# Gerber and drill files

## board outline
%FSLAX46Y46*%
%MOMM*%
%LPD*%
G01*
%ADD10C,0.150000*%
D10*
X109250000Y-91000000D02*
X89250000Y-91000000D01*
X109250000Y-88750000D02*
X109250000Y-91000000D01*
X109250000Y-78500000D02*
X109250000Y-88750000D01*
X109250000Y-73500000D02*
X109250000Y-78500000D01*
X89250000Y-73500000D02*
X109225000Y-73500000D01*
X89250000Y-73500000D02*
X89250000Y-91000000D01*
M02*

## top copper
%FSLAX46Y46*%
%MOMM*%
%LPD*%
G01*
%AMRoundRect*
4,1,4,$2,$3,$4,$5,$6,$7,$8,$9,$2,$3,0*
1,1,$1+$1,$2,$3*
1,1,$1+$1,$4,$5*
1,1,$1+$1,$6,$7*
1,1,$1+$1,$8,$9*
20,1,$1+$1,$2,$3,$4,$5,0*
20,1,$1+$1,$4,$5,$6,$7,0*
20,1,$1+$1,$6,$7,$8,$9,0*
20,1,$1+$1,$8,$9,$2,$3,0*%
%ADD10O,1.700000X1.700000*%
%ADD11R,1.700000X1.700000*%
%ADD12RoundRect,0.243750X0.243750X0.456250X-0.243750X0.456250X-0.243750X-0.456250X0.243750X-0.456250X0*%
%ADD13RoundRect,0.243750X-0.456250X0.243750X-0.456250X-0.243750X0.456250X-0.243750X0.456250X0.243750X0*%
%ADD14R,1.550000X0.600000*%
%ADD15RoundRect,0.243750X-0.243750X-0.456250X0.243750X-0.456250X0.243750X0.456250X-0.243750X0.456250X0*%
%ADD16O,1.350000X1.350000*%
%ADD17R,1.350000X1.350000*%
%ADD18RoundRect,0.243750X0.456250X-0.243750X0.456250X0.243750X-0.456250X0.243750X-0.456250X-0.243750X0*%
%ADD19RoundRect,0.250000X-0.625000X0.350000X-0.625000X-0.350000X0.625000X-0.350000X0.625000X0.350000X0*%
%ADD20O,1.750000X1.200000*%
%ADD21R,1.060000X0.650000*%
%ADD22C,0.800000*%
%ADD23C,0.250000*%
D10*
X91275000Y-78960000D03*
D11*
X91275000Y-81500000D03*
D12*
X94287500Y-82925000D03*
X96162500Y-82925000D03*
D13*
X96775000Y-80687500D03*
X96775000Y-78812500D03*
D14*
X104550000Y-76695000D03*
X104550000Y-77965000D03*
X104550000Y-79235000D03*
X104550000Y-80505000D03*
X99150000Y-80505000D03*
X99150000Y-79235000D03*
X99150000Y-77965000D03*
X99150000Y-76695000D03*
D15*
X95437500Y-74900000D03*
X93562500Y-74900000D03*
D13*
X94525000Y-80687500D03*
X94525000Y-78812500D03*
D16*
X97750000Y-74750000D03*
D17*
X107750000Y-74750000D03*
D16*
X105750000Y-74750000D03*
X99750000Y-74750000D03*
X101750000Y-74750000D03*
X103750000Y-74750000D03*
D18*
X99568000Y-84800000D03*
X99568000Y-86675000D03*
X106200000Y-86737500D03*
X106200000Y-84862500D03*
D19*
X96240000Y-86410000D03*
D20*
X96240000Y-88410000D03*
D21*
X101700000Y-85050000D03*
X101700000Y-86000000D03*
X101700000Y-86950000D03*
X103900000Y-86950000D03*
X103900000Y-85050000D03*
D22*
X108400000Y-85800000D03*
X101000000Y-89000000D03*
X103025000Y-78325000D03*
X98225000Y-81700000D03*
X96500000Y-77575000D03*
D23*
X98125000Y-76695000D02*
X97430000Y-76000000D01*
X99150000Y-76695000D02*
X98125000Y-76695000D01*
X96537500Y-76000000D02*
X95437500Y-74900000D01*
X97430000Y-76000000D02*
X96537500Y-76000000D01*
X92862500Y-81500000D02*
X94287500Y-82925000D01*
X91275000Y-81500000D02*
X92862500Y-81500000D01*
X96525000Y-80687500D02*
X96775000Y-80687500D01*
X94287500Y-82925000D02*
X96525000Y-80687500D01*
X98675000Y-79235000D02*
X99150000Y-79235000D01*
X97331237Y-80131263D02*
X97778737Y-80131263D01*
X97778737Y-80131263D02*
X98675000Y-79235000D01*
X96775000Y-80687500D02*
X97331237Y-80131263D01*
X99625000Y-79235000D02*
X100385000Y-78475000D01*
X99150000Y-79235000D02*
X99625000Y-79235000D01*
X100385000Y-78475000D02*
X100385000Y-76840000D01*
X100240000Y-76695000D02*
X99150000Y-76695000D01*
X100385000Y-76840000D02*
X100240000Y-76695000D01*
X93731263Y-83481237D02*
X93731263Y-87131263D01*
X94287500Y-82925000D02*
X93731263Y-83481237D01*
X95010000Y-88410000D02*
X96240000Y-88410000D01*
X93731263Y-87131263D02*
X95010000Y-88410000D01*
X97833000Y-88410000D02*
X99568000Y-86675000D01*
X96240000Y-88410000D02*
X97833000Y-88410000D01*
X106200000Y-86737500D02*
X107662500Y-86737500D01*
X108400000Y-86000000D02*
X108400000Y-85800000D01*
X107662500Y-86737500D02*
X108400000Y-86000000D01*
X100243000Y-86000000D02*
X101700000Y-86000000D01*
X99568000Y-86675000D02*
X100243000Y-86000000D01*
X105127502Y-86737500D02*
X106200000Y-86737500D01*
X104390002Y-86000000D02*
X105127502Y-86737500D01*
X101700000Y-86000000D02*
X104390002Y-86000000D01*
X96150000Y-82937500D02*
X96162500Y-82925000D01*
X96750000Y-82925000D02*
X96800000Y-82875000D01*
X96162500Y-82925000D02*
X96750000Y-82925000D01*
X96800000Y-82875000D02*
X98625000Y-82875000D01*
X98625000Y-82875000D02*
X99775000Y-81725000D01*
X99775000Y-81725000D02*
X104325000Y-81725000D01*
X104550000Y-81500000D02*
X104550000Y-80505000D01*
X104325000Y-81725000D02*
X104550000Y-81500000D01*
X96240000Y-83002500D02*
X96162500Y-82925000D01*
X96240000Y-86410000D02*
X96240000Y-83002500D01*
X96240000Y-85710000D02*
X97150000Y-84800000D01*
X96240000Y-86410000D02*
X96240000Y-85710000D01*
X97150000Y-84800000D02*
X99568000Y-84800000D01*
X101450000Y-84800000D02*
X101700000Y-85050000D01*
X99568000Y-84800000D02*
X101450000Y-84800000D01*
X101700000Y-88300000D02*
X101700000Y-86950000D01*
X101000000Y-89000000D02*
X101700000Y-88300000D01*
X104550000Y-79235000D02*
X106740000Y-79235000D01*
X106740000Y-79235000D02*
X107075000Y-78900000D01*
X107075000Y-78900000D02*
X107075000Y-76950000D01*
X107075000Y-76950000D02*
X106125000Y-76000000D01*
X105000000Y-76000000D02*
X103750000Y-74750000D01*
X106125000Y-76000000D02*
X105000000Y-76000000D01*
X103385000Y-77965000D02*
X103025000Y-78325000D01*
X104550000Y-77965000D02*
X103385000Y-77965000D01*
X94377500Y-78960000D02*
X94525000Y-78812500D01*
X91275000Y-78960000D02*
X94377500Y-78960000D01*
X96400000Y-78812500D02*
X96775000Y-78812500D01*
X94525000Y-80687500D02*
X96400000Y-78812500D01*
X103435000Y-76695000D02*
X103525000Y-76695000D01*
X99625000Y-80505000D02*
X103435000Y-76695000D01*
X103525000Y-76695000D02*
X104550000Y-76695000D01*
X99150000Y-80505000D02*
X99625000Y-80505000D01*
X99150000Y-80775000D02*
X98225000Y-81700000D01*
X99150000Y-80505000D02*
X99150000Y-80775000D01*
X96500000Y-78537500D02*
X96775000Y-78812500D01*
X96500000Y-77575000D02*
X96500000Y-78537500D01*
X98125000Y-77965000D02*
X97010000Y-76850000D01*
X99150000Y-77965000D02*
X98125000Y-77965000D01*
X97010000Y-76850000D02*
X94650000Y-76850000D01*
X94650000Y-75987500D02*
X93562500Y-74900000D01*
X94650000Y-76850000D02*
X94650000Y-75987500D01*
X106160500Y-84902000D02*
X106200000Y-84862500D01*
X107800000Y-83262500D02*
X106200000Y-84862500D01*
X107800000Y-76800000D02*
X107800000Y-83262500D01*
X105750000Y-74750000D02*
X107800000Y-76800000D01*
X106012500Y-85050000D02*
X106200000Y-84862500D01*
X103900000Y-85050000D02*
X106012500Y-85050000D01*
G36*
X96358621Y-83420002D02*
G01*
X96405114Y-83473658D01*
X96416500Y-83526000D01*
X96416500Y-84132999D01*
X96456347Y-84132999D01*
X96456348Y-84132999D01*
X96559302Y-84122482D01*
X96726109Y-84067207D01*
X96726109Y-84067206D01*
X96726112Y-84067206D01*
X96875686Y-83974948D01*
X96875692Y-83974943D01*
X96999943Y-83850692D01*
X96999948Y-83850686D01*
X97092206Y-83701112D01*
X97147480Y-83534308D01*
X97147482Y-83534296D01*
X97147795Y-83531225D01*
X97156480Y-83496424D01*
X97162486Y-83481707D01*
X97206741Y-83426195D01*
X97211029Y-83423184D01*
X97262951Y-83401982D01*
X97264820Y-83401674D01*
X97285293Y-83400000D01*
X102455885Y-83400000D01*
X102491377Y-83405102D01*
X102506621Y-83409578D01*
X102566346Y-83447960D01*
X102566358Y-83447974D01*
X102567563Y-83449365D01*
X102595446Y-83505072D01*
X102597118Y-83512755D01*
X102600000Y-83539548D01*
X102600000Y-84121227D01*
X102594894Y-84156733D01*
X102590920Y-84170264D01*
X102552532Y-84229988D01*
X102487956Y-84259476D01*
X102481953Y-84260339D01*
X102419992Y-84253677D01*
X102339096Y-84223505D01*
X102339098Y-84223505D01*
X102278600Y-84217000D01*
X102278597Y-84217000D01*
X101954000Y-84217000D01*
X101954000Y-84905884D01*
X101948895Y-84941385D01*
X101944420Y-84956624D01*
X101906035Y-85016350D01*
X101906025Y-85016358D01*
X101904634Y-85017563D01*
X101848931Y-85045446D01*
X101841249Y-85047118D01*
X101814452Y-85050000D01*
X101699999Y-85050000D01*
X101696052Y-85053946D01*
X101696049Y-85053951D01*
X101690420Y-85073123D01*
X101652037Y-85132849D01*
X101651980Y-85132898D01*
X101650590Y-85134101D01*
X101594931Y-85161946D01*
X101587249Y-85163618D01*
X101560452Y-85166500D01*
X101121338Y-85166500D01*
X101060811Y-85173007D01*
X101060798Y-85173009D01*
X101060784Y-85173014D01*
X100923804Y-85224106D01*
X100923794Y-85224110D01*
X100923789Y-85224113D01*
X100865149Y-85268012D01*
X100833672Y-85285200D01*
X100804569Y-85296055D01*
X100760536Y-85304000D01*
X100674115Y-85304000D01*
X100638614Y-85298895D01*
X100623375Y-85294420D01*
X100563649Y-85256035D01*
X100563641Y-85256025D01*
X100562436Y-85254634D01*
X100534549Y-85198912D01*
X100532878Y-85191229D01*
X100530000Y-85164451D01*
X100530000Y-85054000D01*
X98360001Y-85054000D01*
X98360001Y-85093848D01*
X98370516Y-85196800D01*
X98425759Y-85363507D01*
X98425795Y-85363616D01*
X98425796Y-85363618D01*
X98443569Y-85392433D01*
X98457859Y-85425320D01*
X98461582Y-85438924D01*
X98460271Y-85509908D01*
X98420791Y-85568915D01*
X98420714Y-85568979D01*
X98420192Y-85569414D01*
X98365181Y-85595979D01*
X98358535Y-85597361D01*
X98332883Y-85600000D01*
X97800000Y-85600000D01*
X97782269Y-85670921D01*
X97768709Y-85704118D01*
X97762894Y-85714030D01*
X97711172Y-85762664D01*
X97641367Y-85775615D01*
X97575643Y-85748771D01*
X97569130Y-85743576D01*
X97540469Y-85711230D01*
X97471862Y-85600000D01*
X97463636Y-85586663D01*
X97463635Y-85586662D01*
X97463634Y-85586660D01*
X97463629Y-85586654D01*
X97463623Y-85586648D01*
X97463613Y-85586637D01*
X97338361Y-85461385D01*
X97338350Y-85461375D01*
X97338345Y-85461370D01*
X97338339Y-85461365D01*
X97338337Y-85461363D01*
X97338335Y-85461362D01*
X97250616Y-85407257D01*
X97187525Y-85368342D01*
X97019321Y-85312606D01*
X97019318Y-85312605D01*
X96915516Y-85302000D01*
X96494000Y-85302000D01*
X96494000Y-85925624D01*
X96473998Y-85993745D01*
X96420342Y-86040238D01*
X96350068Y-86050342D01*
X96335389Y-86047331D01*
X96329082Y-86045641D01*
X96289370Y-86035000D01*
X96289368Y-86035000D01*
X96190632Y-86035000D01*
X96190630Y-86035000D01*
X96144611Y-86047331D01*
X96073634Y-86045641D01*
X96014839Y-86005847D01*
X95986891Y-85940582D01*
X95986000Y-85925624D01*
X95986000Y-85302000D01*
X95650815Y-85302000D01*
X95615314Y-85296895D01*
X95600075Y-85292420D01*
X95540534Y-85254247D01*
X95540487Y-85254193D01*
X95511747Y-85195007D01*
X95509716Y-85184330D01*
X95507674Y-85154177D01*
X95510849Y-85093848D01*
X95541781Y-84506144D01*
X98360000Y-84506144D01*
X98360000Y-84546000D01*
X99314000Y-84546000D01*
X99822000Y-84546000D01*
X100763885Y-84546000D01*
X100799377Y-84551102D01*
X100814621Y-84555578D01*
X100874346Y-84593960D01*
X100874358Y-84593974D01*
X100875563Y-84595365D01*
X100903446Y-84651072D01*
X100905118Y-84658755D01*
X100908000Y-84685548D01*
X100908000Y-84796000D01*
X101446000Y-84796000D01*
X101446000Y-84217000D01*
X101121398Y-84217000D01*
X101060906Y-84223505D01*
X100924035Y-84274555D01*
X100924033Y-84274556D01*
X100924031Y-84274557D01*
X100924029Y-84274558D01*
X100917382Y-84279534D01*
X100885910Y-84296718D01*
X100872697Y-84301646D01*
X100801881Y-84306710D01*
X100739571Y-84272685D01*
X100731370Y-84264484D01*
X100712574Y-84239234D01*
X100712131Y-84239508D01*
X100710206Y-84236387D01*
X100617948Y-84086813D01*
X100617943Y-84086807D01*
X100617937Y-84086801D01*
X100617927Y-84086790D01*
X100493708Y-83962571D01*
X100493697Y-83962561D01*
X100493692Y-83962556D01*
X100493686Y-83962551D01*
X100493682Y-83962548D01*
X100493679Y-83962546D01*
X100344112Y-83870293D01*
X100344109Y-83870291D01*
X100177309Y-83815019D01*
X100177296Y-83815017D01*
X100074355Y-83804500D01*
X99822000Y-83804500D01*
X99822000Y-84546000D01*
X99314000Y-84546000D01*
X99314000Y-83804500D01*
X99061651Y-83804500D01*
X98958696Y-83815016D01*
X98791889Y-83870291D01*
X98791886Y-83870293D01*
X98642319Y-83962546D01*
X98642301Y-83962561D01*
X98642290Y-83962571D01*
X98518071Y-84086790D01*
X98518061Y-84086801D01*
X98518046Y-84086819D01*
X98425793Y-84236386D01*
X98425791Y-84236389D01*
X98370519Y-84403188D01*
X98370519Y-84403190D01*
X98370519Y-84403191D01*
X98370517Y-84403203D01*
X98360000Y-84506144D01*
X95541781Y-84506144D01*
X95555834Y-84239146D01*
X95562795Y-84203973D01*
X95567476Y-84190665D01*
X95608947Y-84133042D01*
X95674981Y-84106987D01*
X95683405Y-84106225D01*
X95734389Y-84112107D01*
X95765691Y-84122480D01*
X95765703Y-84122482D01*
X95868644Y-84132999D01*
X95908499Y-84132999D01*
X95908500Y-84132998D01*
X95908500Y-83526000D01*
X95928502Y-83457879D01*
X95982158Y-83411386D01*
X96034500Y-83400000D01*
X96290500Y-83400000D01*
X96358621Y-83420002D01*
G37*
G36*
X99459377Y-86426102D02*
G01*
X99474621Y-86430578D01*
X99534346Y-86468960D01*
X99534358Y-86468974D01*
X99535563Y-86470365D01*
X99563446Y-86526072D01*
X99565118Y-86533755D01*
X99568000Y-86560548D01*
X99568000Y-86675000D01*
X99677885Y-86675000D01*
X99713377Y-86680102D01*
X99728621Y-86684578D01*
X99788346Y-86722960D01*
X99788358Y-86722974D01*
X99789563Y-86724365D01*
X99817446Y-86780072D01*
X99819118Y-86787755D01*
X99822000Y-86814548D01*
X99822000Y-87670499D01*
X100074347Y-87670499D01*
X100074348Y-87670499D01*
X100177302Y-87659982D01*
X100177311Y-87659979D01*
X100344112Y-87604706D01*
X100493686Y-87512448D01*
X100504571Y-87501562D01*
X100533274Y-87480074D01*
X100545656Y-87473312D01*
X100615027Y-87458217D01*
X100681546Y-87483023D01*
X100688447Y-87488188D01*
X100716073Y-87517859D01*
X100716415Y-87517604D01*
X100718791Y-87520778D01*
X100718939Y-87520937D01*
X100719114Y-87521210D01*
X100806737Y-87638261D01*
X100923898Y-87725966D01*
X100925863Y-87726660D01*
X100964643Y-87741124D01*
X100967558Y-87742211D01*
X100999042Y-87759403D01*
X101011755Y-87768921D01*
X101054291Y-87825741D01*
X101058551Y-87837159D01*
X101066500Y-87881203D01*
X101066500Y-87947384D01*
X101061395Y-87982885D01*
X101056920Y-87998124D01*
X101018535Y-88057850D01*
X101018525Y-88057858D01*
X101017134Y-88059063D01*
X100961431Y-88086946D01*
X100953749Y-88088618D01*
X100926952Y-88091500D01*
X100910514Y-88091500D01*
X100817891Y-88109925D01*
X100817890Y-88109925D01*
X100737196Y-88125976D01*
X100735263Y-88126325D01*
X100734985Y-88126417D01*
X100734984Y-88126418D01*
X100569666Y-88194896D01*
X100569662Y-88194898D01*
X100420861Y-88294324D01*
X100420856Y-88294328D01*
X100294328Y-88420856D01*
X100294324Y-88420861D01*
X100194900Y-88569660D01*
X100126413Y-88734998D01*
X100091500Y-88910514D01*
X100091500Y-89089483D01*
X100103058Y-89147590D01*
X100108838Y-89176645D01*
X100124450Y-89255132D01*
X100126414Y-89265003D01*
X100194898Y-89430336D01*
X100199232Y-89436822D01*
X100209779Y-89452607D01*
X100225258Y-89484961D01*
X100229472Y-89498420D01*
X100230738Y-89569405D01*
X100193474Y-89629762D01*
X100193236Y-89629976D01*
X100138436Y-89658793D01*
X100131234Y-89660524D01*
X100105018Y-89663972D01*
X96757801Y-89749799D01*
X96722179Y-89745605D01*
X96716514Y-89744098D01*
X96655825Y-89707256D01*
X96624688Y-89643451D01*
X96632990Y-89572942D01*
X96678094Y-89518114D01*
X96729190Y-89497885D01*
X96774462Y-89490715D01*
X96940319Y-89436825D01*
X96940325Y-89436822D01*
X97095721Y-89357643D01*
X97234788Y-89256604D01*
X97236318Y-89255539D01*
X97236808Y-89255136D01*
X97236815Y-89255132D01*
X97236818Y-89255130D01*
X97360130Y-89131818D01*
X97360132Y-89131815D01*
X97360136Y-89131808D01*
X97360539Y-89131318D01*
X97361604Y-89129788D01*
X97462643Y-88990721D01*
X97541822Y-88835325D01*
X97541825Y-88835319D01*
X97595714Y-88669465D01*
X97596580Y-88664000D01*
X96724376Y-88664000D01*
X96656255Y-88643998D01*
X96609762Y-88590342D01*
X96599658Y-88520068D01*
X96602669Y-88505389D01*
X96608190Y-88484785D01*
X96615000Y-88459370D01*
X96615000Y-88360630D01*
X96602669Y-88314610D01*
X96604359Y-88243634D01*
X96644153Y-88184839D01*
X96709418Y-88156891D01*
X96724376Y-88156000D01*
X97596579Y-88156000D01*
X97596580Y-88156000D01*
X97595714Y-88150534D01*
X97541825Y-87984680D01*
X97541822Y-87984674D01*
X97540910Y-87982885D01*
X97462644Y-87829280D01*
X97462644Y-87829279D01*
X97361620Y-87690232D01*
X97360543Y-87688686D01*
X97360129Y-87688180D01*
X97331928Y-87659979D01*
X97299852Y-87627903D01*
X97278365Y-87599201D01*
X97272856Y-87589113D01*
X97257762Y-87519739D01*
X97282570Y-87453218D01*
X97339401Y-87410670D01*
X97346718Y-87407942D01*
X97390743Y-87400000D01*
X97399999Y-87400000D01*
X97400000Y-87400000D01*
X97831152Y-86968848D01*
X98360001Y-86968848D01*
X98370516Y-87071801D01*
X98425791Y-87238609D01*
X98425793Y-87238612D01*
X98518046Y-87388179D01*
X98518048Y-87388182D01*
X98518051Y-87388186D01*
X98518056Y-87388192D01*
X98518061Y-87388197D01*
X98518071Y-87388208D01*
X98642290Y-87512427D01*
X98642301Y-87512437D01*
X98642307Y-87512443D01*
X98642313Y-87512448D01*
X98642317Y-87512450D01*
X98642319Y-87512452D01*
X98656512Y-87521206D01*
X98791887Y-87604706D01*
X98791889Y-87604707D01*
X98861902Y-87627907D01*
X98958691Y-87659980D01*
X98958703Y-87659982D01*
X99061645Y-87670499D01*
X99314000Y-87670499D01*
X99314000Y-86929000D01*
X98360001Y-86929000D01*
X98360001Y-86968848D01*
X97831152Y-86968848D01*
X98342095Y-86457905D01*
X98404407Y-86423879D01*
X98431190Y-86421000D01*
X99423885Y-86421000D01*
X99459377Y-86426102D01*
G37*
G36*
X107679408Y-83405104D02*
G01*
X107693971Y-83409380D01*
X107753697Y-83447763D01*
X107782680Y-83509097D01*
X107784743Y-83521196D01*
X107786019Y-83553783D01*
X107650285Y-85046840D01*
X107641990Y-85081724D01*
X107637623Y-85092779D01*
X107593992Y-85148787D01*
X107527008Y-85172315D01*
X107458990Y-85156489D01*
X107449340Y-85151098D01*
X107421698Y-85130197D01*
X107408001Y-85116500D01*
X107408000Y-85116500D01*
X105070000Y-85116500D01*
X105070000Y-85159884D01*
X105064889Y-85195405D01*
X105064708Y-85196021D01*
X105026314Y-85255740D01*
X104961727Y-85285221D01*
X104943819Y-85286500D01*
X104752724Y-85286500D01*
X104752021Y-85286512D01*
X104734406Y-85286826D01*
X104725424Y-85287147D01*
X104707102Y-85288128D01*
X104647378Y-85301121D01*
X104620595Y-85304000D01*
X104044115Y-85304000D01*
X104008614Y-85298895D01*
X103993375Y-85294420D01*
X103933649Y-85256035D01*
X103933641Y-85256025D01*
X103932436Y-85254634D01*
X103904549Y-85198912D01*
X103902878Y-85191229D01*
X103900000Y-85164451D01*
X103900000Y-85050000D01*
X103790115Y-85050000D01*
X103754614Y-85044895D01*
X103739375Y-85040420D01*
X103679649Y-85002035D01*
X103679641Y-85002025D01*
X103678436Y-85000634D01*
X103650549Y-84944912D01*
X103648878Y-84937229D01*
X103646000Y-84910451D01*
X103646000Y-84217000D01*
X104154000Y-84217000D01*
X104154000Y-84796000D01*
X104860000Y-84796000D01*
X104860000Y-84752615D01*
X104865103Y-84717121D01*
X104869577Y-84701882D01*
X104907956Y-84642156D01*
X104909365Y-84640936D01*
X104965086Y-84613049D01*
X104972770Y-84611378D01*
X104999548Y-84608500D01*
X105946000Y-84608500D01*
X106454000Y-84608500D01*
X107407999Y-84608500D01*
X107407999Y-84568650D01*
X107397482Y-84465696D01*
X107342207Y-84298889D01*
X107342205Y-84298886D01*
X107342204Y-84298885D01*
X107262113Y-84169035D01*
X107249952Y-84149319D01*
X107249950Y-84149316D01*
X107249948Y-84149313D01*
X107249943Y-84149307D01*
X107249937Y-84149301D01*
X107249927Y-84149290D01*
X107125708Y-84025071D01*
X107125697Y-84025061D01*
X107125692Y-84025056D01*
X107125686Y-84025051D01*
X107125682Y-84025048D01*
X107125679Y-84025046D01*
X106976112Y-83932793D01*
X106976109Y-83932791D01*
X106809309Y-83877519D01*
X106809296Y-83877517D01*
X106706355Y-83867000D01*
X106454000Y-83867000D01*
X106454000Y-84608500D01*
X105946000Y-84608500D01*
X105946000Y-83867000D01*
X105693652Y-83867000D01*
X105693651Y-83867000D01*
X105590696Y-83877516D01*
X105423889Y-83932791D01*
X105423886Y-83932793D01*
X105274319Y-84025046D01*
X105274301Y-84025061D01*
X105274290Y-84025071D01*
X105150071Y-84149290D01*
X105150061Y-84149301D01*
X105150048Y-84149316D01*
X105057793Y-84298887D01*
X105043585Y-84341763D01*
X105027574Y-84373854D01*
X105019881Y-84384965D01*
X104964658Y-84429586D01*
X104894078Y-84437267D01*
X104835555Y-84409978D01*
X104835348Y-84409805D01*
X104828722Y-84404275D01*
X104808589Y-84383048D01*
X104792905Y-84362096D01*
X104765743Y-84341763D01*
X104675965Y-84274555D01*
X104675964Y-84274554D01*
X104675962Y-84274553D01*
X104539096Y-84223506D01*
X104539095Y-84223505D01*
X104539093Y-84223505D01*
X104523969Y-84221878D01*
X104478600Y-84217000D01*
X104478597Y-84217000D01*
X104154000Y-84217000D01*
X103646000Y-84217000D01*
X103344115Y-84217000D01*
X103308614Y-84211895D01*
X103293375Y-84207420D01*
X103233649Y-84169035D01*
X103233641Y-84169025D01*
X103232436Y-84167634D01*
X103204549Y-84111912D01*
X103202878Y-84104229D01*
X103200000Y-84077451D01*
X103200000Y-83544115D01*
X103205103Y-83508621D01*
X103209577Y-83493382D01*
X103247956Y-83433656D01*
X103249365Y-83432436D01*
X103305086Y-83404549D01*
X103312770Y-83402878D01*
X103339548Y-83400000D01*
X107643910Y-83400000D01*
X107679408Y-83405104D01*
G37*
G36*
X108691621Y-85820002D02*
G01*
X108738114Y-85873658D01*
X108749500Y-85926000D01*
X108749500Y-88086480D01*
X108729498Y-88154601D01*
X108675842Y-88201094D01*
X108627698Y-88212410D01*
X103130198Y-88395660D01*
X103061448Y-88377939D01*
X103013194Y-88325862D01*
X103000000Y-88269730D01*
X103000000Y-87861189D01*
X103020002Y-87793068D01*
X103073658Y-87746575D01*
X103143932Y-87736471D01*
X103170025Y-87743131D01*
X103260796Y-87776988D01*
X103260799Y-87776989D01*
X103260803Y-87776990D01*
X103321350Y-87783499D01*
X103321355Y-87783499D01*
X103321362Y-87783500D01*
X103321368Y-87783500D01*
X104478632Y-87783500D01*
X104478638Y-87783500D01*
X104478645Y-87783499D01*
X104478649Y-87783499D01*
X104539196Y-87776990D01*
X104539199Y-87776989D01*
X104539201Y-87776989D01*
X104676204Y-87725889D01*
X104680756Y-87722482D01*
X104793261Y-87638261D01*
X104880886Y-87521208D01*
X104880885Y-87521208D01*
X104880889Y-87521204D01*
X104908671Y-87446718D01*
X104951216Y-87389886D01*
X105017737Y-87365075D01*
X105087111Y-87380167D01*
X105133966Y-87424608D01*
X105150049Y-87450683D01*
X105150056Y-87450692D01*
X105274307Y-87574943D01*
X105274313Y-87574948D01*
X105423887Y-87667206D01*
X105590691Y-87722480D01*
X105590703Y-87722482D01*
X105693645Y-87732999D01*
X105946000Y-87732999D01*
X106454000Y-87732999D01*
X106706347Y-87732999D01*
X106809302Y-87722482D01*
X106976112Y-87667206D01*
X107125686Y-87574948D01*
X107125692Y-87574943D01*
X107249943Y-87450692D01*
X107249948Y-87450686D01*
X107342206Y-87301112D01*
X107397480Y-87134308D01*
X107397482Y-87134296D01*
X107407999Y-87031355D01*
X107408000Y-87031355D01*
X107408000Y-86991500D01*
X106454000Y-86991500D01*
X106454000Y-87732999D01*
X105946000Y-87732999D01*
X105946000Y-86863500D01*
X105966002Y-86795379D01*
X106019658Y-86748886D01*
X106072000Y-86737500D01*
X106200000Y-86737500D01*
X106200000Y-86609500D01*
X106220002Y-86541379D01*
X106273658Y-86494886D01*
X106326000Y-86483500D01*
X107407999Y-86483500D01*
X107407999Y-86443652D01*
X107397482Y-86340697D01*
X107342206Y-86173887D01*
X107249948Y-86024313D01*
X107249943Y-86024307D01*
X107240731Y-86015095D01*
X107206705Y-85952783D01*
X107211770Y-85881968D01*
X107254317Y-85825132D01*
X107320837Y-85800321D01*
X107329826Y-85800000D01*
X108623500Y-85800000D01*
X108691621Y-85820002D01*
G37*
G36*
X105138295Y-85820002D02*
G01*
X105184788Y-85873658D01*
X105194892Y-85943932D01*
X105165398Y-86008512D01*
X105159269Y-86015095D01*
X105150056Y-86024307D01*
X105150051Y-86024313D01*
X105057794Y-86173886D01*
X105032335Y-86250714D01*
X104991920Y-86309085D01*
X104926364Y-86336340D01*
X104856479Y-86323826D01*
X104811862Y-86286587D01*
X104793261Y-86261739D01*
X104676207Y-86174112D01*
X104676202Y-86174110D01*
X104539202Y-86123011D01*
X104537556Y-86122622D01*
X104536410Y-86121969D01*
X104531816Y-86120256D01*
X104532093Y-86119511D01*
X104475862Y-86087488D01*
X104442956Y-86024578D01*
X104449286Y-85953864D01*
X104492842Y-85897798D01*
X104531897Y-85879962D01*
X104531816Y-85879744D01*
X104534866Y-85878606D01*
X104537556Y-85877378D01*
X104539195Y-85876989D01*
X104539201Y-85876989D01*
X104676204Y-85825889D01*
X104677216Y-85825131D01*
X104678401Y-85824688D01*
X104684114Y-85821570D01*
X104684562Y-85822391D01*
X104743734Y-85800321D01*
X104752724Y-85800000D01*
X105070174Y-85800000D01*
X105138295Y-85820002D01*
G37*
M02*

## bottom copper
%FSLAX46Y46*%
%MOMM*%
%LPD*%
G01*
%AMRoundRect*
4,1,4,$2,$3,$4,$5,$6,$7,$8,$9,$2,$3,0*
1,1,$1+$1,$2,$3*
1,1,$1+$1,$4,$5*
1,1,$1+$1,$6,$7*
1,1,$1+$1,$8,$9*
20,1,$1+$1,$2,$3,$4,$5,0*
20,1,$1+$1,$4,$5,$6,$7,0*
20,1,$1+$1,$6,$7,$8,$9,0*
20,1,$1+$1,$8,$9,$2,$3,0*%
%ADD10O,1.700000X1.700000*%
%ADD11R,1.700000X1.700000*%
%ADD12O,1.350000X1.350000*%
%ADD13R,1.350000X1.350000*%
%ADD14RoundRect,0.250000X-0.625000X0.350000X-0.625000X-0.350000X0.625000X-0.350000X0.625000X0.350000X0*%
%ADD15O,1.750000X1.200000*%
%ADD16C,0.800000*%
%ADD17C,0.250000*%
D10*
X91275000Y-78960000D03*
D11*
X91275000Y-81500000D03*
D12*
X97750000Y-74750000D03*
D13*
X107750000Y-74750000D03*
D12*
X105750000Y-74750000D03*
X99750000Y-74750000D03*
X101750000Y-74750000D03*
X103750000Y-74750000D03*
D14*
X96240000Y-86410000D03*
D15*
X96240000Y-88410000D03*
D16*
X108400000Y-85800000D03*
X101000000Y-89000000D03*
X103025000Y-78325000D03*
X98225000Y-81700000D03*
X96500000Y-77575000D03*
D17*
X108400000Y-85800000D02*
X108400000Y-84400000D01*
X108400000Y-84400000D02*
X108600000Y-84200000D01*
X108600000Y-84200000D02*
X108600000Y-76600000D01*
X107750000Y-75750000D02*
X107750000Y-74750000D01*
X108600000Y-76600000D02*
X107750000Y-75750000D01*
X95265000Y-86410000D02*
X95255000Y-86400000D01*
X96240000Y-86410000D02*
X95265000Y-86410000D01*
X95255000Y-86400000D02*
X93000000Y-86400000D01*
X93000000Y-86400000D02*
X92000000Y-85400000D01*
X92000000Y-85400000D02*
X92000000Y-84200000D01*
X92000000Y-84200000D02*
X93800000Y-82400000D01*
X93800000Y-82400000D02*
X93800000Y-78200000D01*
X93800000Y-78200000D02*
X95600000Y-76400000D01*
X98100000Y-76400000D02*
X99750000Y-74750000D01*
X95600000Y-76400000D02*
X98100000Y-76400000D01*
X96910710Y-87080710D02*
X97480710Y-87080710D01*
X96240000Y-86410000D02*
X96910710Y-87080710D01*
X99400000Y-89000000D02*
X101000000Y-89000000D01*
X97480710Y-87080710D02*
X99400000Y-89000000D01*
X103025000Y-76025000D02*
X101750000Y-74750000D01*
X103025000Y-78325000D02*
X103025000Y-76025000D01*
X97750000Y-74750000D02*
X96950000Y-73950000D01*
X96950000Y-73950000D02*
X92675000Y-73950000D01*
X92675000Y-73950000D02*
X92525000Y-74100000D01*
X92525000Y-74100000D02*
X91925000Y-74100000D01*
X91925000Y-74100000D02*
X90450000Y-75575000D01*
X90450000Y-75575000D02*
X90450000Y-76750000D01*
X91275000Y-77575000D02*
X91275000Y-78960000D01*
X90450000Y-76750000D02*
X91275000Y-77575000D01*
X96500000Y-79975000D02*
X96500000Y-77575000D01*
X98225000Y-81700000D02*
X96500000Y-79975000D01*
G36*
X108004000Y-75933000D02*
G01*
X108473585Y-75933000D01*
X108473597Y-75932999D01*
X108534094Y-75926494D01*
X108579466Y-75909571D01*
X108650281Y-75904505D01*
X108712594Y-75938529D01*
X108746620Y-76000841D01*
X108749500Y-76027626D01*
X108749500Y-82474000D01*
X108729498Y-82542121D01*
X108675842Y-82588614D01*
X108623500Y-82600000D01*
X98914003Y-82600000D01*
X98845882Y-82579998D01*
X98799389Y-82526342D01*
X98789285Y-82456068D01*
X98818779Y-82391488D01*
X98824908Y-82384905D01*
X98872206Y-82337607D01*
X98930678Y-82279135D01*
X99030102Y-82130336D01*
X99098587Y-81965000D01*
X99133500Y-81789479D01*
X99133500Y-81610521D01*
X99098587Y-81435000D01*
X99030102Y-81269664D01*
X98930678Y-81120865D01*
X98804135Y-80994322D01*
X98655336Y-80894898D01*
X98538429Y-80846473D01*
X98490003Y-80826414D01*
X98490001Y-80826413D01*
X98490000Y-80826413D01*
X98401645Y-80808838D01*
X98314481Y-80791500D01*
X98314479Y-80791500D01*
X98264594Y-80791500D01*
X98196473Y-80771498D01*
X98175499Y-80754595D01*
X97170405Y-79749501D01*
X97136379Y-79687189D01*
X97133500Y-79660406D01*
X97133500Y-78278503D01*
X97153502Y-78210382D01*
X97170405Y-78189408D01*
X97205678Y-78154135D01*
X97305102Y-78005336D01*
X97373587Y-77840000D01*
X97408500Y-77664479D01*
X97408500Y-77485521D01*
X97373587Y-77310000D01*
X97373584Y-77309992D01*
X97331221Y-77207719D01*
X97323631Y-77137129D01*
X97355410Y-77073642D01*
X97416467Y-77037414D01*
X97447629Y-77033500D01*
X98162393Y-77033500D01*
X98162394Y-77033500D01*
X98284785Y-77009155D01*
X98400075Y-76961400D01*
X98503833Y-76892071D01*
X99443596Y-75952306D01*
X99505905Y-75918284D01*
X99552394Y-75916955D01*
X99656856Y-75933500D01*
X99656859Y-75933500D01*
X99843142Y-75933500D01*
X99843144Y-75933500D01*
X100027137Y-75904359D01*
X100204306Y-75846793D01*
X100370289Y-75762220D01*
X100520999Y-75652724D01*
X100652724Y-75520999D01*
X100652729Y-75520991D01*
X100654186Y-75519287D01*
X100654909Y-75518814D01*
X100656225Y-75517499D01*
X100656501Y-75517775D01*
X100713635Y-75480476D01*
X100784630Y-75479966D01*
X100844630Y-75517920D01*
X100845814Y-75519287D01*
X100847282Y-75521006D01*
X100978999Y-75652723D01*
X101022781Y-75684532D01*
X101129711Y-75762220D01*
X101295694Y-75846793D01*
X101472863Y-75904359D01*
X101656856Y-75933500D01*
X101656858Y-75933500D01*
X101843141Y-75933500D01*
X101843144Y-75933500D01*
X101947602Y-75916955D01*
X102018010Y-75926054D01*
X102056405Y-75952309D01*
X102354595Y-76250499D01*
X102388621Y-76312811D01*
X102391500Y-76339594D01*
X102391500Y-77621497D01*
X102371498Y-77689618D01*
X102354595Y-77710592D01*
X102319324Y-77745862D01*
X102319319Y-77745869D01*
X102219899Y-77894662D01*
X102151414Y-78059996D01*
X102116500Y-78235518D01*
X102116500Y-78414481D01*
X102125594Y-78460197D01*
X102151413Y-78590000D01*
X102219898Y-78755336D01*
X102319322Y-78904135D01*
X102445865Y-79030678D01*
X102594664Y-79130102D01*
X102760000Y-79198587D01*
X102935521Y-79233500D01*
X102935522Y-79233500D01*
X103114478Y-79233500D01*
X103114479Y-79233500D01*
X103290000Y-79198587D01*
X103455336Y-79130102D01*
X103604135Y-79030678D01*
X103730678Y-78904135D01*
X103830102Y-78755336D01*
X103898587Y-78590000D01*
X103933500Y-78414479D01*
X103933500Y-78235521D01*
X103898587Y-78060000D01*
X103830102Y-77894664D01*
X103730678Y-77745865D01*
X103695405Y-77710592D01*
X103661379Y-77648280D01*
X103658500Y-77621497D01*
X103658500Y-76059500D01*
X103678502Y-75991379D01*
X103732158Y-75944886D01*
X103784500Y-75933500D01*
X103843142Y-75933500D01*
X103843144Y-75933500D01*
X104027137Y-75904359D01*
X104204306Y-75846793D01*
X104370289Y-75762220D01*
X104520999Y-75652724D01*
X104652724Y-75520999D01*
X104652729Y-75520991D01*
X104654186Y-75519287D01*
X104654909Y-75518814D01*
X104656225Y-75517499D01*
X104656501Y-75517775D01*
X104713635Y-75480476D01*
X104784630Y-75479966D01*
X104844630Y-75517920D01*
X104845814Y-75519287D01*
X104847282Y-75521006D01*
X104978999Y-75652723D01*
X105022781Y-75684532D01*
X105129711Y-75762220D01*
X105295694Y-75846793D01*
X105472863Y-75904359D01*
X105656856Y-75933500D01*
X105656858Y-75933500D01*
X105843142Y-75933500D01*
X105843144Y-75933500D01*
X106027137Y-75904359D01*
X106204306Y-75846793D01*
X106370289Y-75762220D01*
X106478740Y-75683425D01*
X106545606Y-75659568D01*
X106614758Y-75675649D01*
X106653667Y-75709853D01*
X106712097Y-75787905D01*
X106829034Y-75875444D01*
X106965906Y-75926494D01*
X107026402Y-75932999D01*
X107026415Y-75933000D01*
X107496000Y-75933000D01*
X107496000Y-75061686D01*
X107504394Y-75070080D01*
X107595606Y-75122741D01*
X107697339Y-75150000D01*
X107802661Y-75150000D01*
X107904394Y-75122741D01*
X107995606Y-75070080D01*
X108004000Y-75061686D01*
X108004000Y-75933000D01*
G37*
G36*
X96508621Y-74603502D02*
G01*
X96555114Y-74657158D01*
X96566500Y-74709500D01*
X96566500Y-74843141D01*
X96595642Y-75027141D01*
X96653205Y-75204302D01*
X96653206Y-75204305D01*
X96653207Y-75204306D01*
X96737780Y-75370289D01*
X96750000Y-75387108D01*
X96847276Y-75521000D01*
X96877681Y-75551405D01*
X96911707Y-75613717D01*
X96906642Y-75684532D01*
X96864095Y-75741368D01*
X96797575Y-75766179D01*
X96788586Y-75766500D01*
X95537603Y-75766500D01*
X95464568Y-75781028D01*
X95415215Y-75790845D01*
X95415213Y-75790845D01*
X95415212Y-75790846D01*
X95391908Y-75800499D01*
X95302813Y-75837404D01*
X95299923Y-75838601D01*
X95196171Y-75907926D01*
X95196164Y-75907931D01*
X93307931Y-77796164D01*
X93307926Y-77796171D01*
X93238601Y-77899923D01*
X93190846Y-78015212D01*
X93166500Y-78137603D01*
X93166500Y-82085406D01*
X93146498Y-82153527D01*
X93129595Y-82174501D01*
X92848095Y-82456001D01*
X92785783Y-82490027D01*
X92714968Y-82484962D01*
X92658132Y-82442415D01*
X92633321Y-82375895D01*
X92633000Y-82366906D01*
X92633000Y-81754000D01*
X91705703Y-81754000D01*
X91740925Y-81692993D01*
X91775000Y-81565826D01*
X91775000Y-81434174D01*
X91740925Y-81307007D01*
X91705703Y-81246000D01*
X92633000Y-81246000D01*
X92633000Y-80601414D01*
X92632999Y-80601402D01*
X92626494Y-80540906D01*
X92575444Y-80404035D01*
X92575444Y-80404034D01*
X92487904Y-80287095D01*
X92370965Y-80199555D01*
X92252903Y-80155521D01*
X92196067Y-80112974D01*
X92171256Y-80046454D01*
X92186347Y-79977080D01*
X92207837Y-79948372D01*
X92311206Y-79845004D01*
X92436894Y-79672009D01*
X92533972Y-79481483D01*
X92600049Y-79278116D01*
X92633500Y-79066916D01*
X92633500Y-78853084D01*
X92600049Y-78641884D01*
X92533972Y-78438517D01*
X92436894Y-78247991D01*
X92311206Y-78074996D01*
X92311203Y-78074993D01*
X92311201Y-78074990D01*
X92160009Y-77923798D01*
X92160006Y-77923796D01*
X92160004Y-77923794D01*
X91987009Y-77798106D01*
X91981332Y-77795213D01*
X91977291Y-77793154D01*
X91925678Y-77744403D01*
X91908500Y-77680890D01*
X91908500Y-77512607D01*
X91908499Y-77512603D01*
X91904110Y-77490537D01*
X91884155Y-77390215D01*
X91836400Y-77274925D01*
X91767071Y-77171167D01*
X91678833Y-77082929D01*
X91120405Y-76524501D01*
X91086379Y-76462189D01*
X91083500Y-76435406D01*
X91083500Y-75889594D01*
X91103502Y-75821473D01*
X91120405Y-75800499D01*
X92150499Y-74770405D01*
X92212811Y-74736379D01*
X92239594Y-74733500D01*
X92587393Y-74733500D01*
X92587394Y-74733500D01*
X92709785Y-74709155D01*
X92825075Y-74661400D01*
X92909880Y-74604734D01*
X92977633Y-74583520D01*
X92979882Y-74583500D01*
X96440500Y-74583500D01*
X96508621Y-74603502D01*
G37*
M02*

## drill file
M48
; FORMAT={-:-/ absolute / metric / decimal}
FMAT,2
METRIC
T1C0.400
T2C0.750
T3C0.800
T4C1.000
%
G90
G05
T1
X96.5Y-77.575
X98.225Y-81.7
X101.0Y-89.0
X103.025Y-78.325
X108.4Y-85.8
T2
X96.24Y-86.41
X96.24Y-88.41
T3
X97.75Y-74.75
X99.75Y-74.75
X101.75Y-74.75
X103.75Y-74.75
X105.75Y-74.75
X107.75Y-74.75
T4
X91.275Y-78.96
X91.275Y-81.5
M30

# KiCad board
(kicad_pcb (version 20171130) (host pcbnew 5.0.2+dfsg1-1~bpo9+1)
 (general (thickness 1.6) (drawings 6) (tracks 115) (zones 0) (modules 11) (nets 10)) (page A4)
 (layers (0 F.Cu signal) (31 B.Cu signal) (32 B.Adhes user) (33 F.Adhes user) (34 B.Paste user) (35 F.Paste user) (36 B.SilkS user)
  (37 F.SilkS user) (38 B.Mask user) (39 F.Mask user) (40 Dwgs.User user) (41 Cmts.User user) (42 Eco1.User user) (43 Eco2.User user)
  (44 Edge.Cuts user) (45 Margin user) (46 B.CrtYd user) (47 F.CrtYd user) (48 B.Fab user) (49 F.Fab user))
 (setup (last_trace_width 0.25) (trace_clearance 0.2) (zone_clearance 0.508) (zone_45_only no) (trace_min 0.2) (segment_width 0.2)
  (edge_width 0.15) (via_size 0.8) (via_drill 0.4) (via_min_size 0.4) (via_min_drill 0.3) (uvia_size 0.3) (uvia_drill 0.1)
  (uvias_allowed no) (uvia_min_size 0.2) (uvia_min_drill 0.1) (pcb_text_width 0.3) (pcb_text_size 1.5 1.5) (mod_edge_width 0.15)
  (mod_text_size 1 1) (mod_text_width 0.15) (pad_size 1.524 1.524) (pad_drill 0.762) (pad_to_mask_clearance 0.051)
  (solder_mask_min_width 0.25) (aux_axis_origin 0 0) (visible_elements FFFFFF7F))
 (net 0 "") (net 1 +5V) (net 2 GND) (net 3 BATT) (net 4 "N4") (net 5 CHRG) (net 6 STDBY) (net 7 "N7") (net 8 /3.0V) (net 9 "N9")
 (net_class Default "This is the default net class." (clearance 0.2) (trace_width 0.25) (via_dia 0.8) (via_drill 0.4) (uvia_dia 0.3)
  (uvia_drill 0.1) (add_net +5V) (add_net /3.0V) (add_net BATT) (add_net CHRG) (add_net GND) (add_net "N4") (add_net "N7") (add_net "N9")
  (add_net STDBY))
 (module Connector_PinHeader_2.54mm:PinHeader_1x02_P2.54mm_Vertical (layer F.Cu) (at 91.275 81.5 180)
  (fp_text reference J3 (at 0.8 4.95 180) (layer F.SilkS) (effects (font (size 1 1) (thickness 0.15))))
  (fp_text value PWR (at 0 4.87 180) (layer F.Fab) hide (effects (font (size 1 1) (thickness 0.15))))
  (pad 2 thru_hole oval (at 0 2.54 180) (size 1.7 1.7) (drill 1) (layers *.Cu *.Mask) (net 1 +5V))
  (pad 1 thru_hole rect (at 0 0 180) (size 1.7 1.7) (drill 1) (layers *.Cu *.Mask) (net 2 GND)))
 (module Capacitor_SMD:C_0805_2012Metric (layer F.Cu) (at 95.225 82.925 180)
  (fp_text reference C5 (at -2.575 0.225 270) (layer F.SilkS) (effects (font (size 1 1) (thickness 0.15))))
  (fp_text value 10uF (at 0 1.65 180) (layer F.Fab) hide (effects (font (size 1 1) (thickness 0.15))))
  (pad 2 smd roundrect (at 0.9375 0 180) (size 0.975 1.4) (layers F.Cu F.Paste F.Mask) (roundrect_rratio 0.25) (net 2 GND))
  (pad 1 smd roundrect (at -0.9375 0 180) (size 0.975 1.4) (layers F.Cu F.Paste F.Mask) (roundrect_rratio 0.25) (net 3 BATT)))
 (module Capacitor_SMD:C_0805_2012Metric (layer F.Cu) (at 96.775 79.75 270)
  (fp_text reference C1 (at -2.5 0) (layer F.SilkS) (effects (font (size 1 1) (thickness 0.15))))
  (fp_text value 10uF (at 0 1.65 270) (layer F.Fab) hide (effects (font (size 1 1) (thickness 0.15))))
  (pad 2 smd roundrect (at 0.9375 0 270) (size 0.975 1.4) (layers F.Cu F.Paste F.Mask) (roundrect_rratio 0.25) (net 2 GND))
  (pad 1 smd roundrect (at -0.9375 0 270) (size 0.975 1.4) (layers F.Cu F.Paste F.Mask) (roundrect_rratio 0.25) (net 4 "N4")))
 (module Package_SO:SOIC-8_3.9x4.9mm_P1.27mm (layer F.Cu) (at 101.85 78.6)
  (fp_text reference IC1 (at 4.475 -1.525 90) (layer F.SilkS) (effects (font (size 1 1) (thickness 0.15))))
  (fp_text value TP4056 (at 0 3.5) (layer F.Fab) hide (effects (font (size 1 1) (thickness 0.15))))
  (pad 8 smd rect (at 2.7 -1.905) (size 1.55 0.6) (layers F.Cu F.Paste F.Mask) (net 4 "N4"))
  (pad 7 smd rect (at 2.7 -0.635) (size 1.55 0.6) (layers F.Cu F.Paste F.Mask) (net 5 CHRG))
  (pad 6 smd rect (at 2.7 0.635) (size 1.55 0.6) (layers F.Cu F.Paste F.Mask) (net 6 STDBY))
  (pad 5 smd rect (at 2.7 1.905) (size 1.55 0.6) (layers F.Cu F.Paste F.Mask) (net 3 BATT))
  (pad 4 smd rect (at -2.7 1.905) (size 1.55 0.6) (layers F.Cu F.Paste F.Mask) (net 4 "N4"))
  (pad 3 smd rect (at -2.7 0.635) (size 1.55 0.6) (layers F.Cu F.Paste F.Mask) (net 2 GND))
  (pad 2 smd rect (at -2.7 -0.635) (size 1.55 0.6) (layers F.Cu F.Paste F.Mask) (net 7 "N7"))
  (pad 1 smd rect (at -2.7 -1.905) (size 1.55 0.6) (layers F.Cu F.Paste F.Mask) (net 2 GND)))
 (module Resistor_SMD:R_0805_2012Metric (layer F.Cu) (at 94.5 74.9)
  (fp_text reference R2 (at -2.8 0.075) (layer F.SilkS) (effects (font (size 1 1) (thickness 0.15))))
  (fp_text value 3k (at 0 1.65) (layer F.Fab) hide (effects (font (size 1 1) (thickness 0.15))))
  (pad 2 smd roundrect (at 0.9375 0) (size 0.975 1.4) (layers F.Cu F.Paste F.Mask) (roundrect_rratio 0.25) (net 2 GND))
  (pad 1 smd roundrect (at -0.9375 0) (size 0.975 1.4) (layers F.Cu F.Paste F.Mask) (roundrect_rratio 0.25) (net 7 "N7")))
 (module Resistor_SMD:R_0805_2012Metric (layer F.Cu) (at 94.525 79.75 270)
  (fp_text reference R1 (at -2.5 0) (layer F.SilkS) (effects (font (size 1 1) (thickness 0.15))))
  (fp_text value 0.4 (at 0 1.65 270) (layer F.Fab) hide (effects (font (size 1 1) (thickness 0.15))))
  (pad 2 smd roundrect (at 0.9375 0 270) (size 0.975 1.4) (layers F.Cu F.Paste F.Mask) (roundrect_rratio 0.25) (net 4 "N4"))
  (pad 1 smd roundrect (at -0.9375 0 270) (size 0.975 1.4) (layers F.Cu F.Paste F.Mask) (roundrect_rratio 0.25) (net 1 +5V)))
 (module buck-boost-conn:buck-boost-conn (layer F.Cu) (at 102.75 79.75)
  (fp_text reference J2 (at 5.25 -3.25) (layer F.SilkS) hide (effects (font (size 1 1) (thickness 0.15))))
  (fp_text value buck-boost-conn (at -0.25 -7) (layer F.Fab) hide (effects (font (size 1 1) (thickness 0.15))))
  (pad 6 thru_hole oval (at -5 -5) (size 1.35 1.35) (drill 0.8) (layers *.Cu *.Mask) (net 1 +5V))
  (pad 1 thru_hole rect (at 5 -5) (size 1.35 1.35) (drill 0.8) (layers *.Cu *.Mask) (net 2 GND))
  (pad 2 thru_hole oval (at 3 -5) (size 1.35 1.35) (drill 0.8) (layers *.Cu *.Mask) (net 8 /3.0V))
  (pad 3 thru_hole oval (at -3 -5) (size 1.35 1.35) (drill 0.8) (layers *.Cu *.Mask) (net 3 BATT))
  (pad 4 thru_hole oval (at -1 -5) (size 1.35 1.35) (drill 0.8) (layers *.Cu *.Mask) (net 5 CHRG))
  (pad 5 thru_hole oval (at 1 -5) (size 1.35 1.35) (drill 0.8) (layers *.Cu *.Mask) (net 6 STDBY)))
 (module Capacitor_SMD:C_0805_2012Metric (layer F.Cu) (at 99.568 85.7375 90)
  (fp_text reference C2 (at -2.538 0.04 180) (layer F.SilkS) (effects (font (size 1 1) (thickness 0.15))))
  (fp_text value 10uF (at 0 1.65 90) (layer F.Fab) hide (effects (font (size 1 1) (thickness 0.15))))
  (pad 2 smd roundrect (at 0.9375 0 90) (size 0.975 1.4) (layers F.Cu F.Paste F.Mask) (roundrect_rratio 0.25) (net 3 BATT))
  (pad 1 smd roundrect (at -0.9375 0 90) (size 0.975 1.4) (layers F.Cu F.Paste F.Mask) (roundrect_rratio 0.25) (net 2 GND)))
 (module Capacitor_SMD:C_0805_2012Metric (layer F.Cu) (at 106.2 85.8 90)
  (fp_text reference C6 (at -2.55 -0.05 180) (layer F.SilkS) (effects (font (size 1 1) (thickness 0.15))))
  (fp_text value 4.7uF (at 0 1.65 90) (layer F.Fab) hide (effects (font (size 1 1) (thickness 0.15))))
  (pad 1 smd roundrect (at -0.9375 0 90) (size 0.975 1.4) (layers F.Cu F.Paste F.Mask) (roundrect_rratio 0.25) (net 2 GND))
  (pad 2 smd roundrect (at 0.9375 0 90) (size 0.975 1.4) (layers F.Cu F.Paste F.Mask) (roundrect_rratio 0.25) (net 8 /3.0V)))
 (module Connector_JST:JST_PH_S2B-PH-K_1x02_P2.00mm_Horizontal (layer F.Cu) (at 96.24 86.41 270)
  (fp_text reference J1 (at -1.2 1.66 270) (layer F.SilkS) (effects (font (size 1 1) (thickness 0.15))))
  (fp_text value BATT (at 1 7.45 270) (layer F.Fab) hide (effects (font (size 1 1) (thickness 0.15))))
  (pad 1 thru_hole roundrect (at 0 0 270) (size 1.2 1.75) (drill 0.75) (layers *.Cu *.Mask) (roundrect_rratio 0.208333) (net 3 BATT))
  (pad 2 thru_hole oval (at 2 0 270) (size 1.2 1.75) (drill 0.75) (layers *.Cu *.Mask) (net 2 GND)))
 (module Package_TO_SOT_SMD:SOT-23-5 (layer F.Cu) (at 102.8 86)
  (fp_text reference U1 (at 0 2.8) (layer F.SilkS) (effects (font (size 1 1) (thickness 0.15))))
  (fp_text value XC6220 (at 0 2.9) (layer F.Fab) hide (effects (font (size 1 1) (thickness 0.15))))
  (pad 1 smd rect (at -1.1 -0.95) (size 1.06 0.65) (layers F.Cu F.Paste F.Mask) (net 3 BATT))
  (pad 2 smd rect (at -1.1 0) (size 1.06 0.65) (layers F.Cu F.Paste F.Mask) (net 2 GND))
  (pad 3 smd rect (at -1.1 0.95) (size 1.06 0.65) (layers F.Cu F.Paste F.Mask) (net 3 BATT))
  (pad 4 smd rect (at 1.1 0.95) (size 1.06 0.65) (layers F.Cu F.Paste F.Mask) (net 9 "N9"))
  (pad 5 smd rect (at 1.1 -0.95) (size 1.06 0.65) (layers F.Cu F.Paste F.Mask) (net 8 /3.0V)))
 (gr_line (start 109.25 91) (end 89.25 91) (layer Edge.Cuts) (width 0.15))
 (gr_line (start 109.25 88.75) (end 109.25 91) (layer Edge.Cuts) (width 0.15))
 (gr_line (start 109.25 78.5) (end 109.25 88.75) (layer Edge.Cuts) (width 0.15))
 (gr_line (start 109.25 73.5) (end 109.25 78.5) (layer Edge.Cuts) (width 0.15))
 (gr_line (start 89.25 73.5) (end 109.225 73.5) (layer Edge.Cuts) (width 0.15))
 (gr_line (start 89.25 73.5) (end 89.25 91) (layer Edge.Cuts) (width 0.15))
 (segment (start 98.125 76.695) (end 97.43 76) (width 0.25) (layer F.Cu) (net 2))
 (segment (start 99.15 76.695) (end 98.125 76.695) (width 0.25) (layer F.Cu) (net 2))
 (segment (start 96.5375 76) (end 95.4375 74.9) (width 0.25) (layer F.Cu) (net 2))
 (segment (start 97.43 76) (end 96.5375 76) (width 0.25) (layer F.Cu) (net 2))
 (segment (start 92.8625 81.5) (end 94.2875 82.925) (width 0.25) (layer F.Cu) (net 2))
 (segment (start 91.275 81.5) (end 92.8625 81.5) (width 0.25) (layer F.Cu) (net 2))
 (segment (start 96.525 80.6875) (end 96.775 80.6875) (width 0.25) (layer F.Cu) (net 2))
 (segment (start 94.2875 82.925) (end 96.525 80.6875) (width 0.25) (layer F.Cu) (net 2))
 (segment (start 98.675 79.235) (end 99.15 79.235) (width 0.25) (layer F.Cu) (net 2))
 (segment (start 97.331237 80.131263) (end 97.778737 80.131263) (width 0.25) (layer F.Cu) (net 2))
 (segment (start 97.778737 80.131263) (end 98.675 79.235) (width 0.25) (layer F.Cu) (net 2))
 (segment (start 96.775 80.6875) (end 97.331237 80.131263) (width 0.25) (layer F.Cu) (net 2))
 (segment (start 99.625 79.235) (end 100.385 78.475) (width 0.25) (layer F.Cu) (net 2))
 (segment (start 99.15 79.235) (end 99.625 79.235) (width 0.25) (layer F.Cu) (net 2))
 (segment (start 100.385 78.475) (end 100.385 76.84) (width 0.25) (layer F.Cu) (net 2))
 (segment (start 100.24 76.695) (end 99.15 76.695) (width 0.25) (layer F.Cu) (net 2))
 (segment (start 100.385 76.84) (end 100.24 76.695) (width 0.25) (layer F.Cu) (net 2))
 (segment (start 93.731263 83.481237) (end 93.731263 87.131263) (width 0.25) (layer F.Cu) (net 2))
 (segment (start 94.2875 82.925) (end 93.731263 83.481237) (width 0.25) (layer F.Cu) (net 2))
 (segment (start 95.01 88.41) (end 96.24 88.41) (width 0.25) (layer F.Cu) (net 2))
 (segment (start 93.731263 87.131263) (end 95.01 88.41) (width 0.25) (layer F.Cu) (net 2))
 (segment (start 97.833 88.41) (end 99.568 86.675) (width 0.25) (layer F.Cu) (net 2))
 (segment (start 96.24 88.41) (end 97.833 88.41) (width 0.25) (layer F.Cu) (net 2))
 (segment (start 106.2 86.7375) (end 107.6625 86.7375) (width 0.25) (layer F.Cu) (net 2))
 (segment (start 108.4 86) (end 108.4 85.8) (width 0.25) (layer F.Cu) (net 2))
 (via (at 108.4 85.8) (size 0.8) (drill 0.4) (layers F.Cu B.Cu) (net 2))
 (segment (start 107.6625 86.7375) (end 108.4 86) (width 0.25) (layer F.Cu) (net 2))
 (segment (start 108.4 85.8) (end 108.4 84.4) (width 0.25) (layer B.Cu) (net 2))
 (segment (start 108.4 84.4) (end 108.6 84.2) (width 0.25) (layer B.Cu) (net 2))
 (segment (start 108.6 84.2) (end 108.6 76.6) (width 0.25) (layer B.Cu) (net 2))
 (segment (start 107.75 75.75) (end 107.75 74.75) (width 0.25) (layer B.Cu) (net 2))
 (segment (start 108.6 76.6) (end 107.75 75.75) (width 0.25) (layer B.Cu) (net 2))
 (segment (start 100.243 86) (end 101.7 86) (width 0.25) (layer F.Cu) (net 2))
 (segment (start 99.568 86.675) (end 100.243 86) (width 0.25) (layer F.Cu) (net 2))
 (segment (start 105.127502 86.7375) (end 106.2 86.7375) (width 0.25) (layer F.Cu) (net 2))
 (segment (start 104.390002 86) (end 105.127502 86.7375) (width 0.25) (layer F.Cu) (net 2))
 (segment (start 101.7 86) (end 104.390002 86) (width 0.25) (layer F.Cu) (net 2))
 (segment (start 96.15 82.9375) (end 96.1625 82.925) (width 0.25) (layer F.Cu) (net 3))
 (segment (start 96.75 82.925) (end 96.8 82.875) (width 0.25) (layer F.Cu) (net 3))
 (segment (start 96.1625 82.925) (end 96.75 82.925) (width 0.25) (layer F.Cu) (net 3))
 (segment (start 96.8 82.875) (end 98.625 82.875) (width 0.25) (layer F.Cu) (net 3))
 (segment (start 98.625 82.875) (end 99.775 81.725) (width 0.25) (layer F.Cu) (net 3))
 (segment (start 99.775 81.725) (end 104.325 81.725) (width 0.25) (layer F.Cu) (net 3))
 (segment (start 104.55 81.5) (end 104.55 80.505) (width 0.25) (layer F.Cu) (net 3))
 (segment (start 104.325 81.725) (end 104.55 81.5) (width 0.25) (layer F.Cu) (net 3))
 (segment (start 96.24 83.0025) (end 96.1625 82.925) (width 0.25) (layer F.Cu) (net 3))
 (segment (start 96.24 86.41) (end 96.24 83.0025) (width 0.25) (layer F.Cu) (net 3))
 (segment (start 95.265 86.41) (end 95.255 86.4) (width 0.25) (layer B.Cu) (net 3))
 (segment (start 96.24 86.41) (end 95.265 86.41) (width 0.25) (layer B.Cu) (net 3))
 (segment (start 95.255 86.4) (end 93 86.4) (width 0.25) (layer B.Cu) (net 3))
 (segment (start 93 86.4) (end 92 85.4) (width 0.25) (layer B.Cu) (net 3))
 (segment (start 92 85.4) (end 92 84.2) (width 0.25) (layer B.Cu) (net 3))
 (segment (start 92 84.2) (end 93.8 82.4) (width 0.25) (layer B.Cu) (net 3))
 (segment (start 93.8 82.4) (end 93.8 78.2) (width 0.25) (layer B.Cu) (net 3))
 (segment (start 93.8 78.2) (end 95.6 76.4) (width 0.25) (layer B.Cu) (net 3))
 (segment (start 98.1 76.4) (end 99.75 74.75) (width 0.25) (layer B.Cu) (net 3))
 (segment (start 95.6 76.4) (end 98.1 76.4) (width 0.25) (layer B.Cu) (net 3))
 (segment (start 96.24 85.71) (end 97.15 84.8) (width 0.25) (layer F.Cu) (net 3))
 (segment (start 96.24 86.41) (end 96.24 85.71) (width 0.25) (layer F.Cu) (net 3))
 (segment (start 97.15 84.8) (end 99.568 84.8) (width 0.25) (layer F.Cu) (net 3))
 (segment (start 101.45 84.8) (end 101.7 85.05) (width 0.25) (layer F.Cu) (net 3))
 (segment (start 99.568 84.8) (end 101.45 84.8) (width 0.25) (layer F.Cu) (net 3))
 (segment (start 96.91071 87.08071) (end 97.48071 87.08071) (width 0.25) (layer B.Cu) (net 3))
 (segment (start 96.24 86.41) (end 96.91071 87.08071) (width 0.25) (layer B.Cu) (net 3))
 (via (at 101 89) (size 0.8) (drill 0.4) (layers F.Cu B.Cu) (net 3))
 (segment (start 99.4 89) (end 101 89) (width 0.25) (layer B.Cu) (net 3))
 (segment (start 97.48071 87.08071) (end 99.4 89) (width 0.25) (layer B.Cu) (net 3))
 (segment (start 101.7 88.3) (end 101.7 86.95) (width 0.25) (layer F.Cu) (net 3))
 (segment (start 101 89) (end 101.7 88.3) (width 0.25) (layer F.Cu) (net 3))
 (segment (start 104.55 79.235) (end 106.74 79.235) (width 0.25) (layer F.Cu) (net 6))
 (segment (start 106.74 79.235) (end 107.075 78.9) (width 0.25) (layer F.Cu) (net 6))
 (segment (start 107.075 78.9) (end 107.075 76.95) (width 0.25) (layer F.Cu) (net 6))
 (segment (start 107.075 76.95) (end 106.125 76) (width 0.25) (layer F.Cu) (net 6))
 (segment (start 105 76) (end 103.75 74.75) (width 0.25) (layer F.Cu) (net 6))
 (segment (start 106.125 76) (end 105 76) (width 0.25) (layer F.Cu) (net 6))
 (via (at 103.025 78.325) (size 0.8) (drill 0.4) (layers F.Cu B.Cu) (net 5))
 (segment (start 103.385 77.965) (end 103.025 78.325) (width 0.25) (layer F.Cu) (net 5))
 (segment (start 104.55 77.965) (end 103.385 77.965) (width 0.25) (layer F.Cu) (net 5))
 (segment (start 103.025 76.025) (end 101.75 74.75) (width 0.25) (layer B.Cu) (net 5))
 (segment (start 103.025 78.325) (end 103.025 76.025) (width 0.25) (layer B.Cu) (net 5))
 (segment (start 97.75 74.75) (end 96.95 73.95) (width 0.25) (layer B.Cu) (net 1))
 (segment (start 96.95 73.95) (end 92.675 73.95) (width 0.25) (layer B.Cu) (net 1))
 (segment (start 92.675 73.95) (end 92.525 74.1) (width 0.25) (layer B.Cu) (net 1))
 (segment (start 92.525 74.1) (end 91.925 74.1) (width 0.25) (layer B.Cu) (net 1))
 (segment (start 91.925 74.1) (end 90.45 75.575) (width 0.25) (layer B.Cu) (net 1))
 (segment (start 90.45 75.575) (end 90.45 76.75) (width 0.25) (layer B.Cu) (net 1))
 (segment (start 91.275 77.575) (end 91.275 78.96) (width 0.25) (layer B.Cu) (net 1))
 (segment (start 90.45 76.75) (end 91.275 77.575) (width 0.25) (layer B.Cu) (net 1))
 (segment (start 94.3775 78.96) (end 94.525 78.8125) (width 0.25) (layer F.Cu) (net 1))
 (segment (start 91.275 78.96) (end 94.3775 78.96) (width 0.25) (layer F.Cu) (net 1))
 (segment (start 96.4 78.8125) (end 96.775 78.8125) (width 0.25) (layer F.Cu) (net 4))
 (segment (start 94.525 80.6875) (end 96.4 78.8125) (width 0.25) (layer F.Cu) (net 4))
 (segment (start 103.435 76.695) (end 103.525 76.695) (width 0.25) (layer F.Cu) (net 4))
 (segment (start 99.625 80.505) (end 103.435 76.695) (width 0.25) (layer F.Cu) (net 4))
 (segment (start 103.525 76.695) (end 104.55 76.695) (width 0.25) (layer F.Cu) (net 4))
 (segment (start 99.15 80.505) (end 99.625 80.505) (width 0.25) (layer F.Cu) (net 4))
 (via (at 98.225 81.7) (size 0.8) (drill 0.4) (layers F.Cu B.Cu) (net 4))
 (segment (start 99.15 80.775) (end 98.225 81.7) (width 0.25) (layer F.Cu) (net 4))
 (segment (start 99.15 80.505) (end 99.15 80.775) (width 0.25) (layer F.Cu) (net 4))
 (via (at 96.5 77.575) (size 0.8) (drill 0.4) (layers F.Cu B.Cu) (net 4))
 (segment (start 96.5 79.975) (end 96.5 77.575) (width 0.25) (layer B.Cu) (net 4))
 (segment (start 98.225 81.7) (end 96.5 79.975) (width 0.25) (layer B.Cu) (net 4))
 (segment (start 96.5 78.5375) (end 96.775 78.8125) (width 0.25) (layer F.Cu) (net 4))
 (segment (start 96.5 77.575) (end 96.5 78.5375) (width 0.25) (layer F.Cu) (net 4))
 (segment (start 98.125 77.965) (end 97.01 76.85) (width 0.25) (layer F.Cu) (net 7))
 (segment (start 99.15 77.965) (end 98.125 77.965) (width 0.25) (layer F.Cu) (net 7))
 (segment (start 97.01 76.85) (end 94.65 76.85) (width 0.25) (layer F.Cu) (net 7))
 (segment (start 94.65 75.9875) (end 93.5625 74.9) (width 0.25) (layer F.Cu) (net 7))
 (segment (start 94.65 76.85) (end 94.65 75.9875) (width 0.25) (layer F.Cu) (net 7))
 (segment (start 106.1605 84.902) (end 106.2 84.8625) (width 0.25) (layer F.Cu) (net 8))
 (segment (start 107.8 83.2625) (end 106.2 84.8625) (width 0.25) (layer F.Cu) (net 8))
 (segment (start 107.8 76.8) (end 107.8 83.2625) (width 0.25) (layer F.Cu) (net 8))
 (segment (start 105.75 74.75) (end 107.8 76.8) (width 0.25) (layer F.Cu) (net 8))
 (segment (start 106.0125 85.05) (end 106.2 84.8625) (width 0.25) (layer F.Cu) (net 8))
 (segment (start 103.9 85.05) (end 106.0125 85.05) (width 0.25) (layer F.Cu) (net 8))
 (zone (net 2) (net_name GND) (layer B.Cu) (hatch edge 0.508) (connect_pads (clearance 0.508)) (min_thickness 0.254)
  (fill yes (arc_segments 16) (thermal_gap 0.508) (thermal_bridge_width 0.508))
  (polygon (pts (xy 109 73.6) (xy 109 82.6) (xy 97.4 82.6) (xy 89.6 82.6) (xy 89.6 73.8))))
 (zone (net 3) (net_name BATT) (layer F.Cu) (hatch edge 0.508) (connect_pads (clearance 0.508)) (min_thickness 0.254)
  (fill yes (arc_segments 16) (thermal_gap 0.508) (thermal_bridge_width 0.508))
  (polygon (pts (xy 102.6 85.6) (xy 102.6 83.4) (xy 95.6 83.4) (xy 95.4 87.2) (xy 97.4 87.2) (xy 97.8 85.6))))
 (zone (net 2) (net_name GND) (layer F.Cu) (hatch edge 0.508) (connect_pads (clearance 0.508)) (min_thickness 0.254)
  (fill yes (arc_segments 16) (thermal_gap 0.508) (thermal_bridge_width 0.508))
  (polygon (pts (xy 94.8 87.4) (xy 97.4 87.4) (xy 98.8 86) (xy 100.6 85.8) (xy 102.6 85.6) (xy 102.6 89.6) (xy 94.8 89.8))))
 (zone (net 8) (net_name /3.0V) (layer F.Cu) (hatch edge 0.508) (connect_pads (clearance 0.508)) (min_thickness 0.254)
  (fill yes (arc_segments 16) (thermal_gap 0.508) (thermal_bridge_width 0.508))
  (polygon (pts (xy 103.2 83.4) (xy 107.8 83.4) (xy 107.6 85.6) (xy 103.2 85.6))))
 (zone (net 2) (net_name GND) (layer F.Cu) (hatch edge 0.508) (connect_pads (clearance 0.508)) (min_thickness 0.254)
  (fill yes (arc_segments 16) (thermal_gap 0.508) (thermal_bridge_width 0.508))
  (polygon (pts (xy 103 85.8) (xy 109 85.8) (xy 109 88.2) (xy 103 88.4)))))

